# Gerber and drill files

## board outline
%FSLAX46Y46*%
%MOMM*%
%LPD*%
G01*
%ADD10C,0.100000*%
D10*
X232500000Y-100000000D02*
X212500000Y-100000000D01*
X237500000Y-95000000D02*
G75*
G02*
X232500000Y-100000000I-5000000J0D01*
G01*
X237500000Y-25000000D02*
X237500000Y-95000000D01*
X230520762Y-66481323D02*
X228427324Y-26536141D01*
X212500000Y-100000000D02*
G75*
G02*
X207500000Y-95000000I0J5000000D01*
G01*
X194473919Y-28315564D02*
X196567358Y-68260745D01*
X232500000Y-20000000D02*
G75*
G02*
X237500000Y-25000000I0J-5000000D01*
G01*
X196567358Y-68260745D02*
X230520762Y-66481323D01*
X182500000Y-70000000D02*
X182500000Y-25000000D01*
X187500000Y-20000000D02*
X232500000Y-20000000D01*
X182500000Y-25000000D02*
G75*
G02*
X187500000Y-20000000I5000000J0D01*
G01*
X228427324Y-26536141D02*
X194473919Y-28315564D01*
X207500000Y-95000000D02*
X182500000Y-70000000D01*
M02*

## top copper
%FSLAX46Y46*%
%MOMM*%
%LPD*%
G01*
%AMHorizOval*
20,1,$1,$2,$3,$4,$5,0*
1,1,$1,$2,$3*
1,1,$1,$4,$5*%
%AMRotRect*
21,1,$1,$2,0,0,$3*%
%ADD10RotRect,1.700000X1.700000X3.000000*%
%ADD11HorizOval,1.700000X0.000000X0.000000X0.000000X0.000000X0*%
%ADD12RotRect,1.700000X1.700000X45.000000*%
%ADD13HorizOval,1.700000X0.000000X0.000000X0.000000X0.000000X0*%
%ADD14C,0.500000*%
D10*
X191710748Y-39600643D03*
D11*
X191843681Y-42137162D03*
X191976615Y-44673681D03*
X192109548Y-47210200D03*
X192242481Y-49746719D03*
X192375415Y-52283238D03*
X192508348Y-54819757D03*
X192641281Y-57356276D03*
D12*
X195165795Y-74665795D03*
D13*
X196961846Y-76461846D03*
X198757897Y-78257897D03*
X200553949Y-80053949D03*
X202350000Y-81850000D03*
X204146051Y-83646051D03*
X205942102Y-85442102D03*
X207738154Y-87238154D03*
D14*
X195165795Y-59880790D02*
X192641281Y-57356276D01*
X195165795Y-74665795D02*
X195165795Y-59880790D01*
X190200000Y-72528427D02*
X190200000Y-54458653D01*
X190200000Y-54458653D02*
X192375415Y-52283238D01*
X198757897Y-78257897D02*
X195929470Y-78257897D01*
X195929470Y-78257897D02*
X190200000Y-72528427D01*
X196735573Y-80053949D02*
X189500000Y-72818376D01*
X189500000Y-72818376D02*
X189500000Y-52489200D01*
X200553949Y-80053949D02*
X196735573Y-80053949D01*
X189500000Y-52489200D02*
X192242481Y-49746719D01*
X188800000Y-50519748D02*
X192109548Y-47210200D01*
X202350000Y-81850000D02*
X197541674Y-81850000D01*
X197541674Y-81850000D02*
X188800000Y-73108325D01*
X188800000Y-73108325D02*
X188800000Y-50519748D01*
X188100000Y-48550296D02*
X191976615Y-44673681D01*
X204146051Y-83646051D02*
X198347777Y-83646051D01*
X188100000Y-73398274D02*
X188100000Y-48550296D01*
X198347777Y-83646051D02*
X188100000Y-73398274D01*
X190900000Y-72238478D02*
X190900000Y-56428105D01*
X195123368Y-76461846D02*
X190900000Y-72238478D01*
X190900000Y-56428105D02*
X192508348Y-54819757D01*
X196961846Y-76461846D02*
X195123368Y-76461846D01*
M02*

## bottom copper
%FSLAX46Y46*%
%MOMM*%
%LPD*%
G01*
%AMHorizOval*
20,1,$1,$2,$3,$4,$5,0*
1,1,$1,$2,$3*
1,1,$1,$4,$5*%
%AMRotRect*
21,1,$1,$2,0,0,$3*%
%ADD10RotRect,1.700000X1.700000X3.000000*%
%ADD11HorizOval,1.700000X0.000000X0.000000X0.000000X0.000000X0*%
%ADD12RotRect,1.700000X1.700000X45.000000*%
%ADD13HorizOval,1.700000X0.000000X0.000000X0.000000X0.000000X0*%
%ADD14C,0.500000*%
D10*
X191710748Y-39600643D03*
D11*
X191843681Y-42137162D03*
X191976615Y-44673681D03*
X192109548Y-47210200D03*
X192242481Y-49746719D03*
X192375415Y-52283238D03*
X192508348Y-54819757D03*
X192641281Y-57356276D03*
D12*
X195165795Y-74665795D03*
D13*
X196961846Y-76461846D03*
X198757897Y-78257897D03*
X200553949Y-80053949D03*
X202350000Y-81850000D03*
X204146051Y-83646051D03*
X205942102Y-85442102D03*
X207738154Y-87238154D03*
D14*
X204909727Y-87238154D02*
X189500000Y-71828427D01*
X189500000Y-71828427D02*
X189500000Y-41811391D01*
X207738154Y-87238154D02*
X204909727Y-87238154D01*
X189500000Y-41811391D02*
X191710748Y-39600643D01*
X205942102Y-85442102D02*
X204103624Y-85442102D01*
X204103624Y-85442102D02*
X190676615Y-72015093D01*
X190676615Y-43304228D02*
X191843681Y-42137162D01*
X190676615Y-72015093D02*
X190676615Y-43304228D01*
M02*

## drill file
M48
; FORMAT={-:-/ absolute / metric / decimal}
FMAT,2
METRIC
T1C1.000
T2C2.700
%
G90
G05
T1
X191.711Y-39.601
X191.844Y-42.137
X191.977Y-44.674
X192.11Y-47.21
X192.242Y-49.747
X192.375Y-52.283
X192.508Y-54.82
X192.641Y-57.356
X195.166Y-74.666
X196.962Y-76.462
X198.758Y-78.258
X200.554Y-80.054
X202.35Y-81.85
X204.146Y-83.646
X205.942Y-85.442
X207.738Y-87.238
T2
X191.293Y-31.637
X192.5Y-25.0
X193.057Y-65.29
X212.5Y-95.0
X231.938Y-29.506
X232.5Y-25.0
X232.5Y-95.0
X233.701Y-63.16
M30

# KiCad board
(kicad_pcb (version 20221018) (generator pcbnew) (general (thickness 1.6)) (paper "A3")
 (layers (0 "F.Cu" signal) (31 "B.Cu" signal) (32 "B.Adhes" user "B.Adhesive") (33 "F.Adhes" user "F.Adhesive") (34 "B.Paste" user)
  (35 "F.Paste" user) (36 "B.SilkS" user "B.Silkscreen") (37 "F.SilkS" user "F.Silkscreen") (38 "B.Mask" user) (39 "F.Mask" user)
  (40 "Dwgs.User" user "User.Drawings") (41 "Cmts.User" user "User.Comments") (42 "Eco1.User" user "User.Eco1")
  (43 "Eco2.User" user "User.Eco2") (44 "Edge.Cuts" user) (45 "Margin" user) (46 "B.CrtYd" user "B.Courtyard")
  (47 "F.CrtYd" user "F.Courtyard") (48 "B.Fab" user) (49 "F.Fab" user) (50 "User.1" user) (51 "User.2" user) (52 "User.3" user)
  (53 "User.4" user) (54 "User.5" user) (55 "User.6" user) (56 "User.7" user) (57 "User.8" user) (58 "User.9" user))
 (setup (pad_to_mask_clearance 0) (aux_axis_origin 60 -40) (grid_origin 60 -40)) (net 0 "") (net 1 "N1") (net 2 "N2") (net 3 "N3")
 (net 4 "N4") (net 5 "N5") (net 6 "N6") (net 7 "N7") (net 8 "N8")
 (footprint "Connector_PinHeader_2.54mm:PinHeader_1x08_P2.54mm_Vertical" (layer "F.Cu") (at 191.710748 39.600643 3)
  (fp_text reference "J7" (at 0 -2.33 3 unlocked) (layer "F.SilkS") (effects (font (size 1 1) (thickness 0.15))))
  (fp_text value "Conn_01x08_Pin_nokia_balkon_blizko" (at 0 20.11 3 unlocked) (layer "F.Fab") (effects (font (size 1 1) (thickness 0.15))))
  (pad "1" thru_hole rect (at 0 0 3) (size 1.7 1.7) (drill 1) (layers "*.Cu" "*.Mask") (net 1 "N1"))
  (pad "2" thru_hole oval (at 0 2.54 3) (size 1.7 1.7) (drill 1) (layers "*.Cu" "*.Mask") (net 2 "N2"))
  (pad "3" thru_hole oval (at 0 5.08 3) (size 1.7 1.7) (drill 1) (layers "*.Cu" "*.Mask") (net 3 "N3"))
  (pad "4" thru_hole oval (at 0 7.62 3) (size 1.7 1.7) (drill 1) (layers "*.Cu" "*.Mask") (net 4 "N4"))
  (pad "5" thru_hole oval (at 0 10.16 3) (size 1.7 1.7) (drill 1) (layers "*.Cu" "*.Mask") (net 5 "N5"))
  (pad "6" thru_hole oval (at 0 12.7 3) (size 1.7 1.7) (drill 1) (layers "*.Cu" "*.Mask") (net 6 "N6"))
  (pad "7" thru_hole oval (at 0 15.24 3) (size 1.7 1.7) (drill 1) (layers "*.Cu" "*.Mask") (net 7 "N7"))
  (pad "8" thru_hole oval (at 0 17.78 3) (size 1.7 1.7) (drill 1) (layers "*.Cu" "*.Mask") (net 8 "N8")))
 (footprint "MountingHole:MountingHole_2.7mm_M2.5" (layer "F.Cu") (at 232.5 25)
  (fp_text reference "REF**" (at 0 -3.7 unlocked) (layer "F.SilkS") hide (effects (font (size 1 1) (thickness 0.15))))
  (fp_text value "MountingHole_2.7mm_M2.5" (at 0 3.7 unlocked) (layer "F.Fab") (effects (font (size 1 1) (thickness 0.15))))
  (pad "" np_thru_hole circle (at 0 0) (size 2.7 2.7) (drill 2.7) (layers "*.Cu" "*.Mask")))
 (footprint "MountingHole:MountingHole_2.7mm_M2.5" (layer "F.Cu") (at 192.5 25)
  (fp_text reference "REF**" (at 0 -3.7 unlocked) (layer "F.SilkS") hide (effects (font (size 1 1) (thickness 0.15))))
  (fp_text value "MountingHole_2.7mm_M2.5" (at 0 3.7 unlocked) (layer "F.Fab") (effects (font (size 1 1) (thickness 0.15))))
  (pad "" np_thru_hole circle (at 0 0) (size 2.7 2.7) (drill 2.7) (layers "*.Cu" "*.Mask")))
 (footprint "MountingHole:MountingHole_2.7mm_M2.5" (layer "F.Cu") (at 191.293369 31.636572 3)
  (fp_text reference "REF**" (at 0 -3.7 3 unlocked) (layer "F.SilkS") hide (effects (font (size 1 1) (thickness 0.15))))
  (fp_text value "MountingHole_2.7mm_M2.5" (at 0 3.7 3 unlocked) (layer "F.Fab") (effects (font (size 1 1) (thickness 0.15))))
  (pad "" np_thru_hole circle (at 0 0 3) (size 2.7 2.7) (drill 2.7) (layers "*.Cu" "*.Mask")))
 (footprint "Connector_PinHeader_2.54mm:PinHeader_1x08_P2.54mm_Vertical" (layer "F.Cu") (at 195.165795 74.665795 45)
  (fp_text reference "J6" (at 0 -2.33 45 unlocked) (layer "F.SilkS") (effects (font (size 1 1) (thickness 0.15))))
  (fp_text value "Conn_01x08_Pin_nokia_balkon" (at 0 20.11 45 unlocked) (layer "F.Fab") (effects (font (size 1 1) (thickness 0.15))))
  (pad "1" thru_hole rect (at 0 0 45) (size 1.7 1.7) (drill 1) (layers "*.Cu" "*.Mask") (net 8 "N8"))
  (pad "2" thru_hole oval (at 0 2.54 45) (size 1.7 1.7) (drill 1) (layers "*.Cu" "*.Mask") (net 7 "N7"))
  (pad "3" thru_hole oval (at 0 5.08 45) (size 1.7 1.7) (drill 1) (layers "*.Cu" "*.Mask") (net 6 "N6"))
  (pad "4" thru_hole oval (at 0 7.62 45) (size 1.7 1.7) (drill 1) (layers "*.Cu" "*.Mask") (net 5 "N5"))
  (pad "5" thru_hole oval (at 0 10.16 45) (size 1.7 1.7) (drill 1) (layers "*.Cu" "*.Mask") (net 4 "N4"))
  (pad "6" thru_hole oval (at 0 12.7 45) (size 1.7 1.7) (drill 1) (layers "*.Cu" "*.Mask") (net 3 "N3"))
  (pad "7" thru_hole oval (at 0 15.24 45) (size 1.7 1.7) (drill 1) (layers "*.Cu" "*.Mask") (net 2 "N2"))
  (pad "8" thru_hole oval (at 0 17.78 45) (size 1.7 1.7) (drill 1) (layers "*.Cu" "*.Mask") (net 1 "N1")))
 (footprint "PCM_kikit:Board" (layer "F.Cu") (at 220.5 100 180)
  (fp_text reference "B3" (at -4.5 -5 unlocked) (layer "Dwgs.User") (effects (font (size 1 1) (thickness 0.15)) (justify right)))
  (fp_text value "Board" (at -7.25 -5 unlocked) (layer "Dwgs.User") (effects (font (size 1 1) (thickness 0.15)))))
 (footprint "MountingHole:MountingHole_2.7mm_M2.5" (layer "F.Cu") (at 232.5 95)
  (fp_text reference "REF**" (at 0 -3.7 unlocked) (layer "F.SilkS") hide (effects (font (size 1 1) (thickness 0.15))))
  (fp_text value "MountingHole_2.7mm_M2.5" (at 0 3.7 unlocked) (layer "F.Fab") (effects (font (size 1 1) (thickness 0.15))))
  (pad "" np_thru_hole circle (at 0 0) (size 2.7 2.7) (drill 2.7) (layers "*.Cu" "*.Mask")))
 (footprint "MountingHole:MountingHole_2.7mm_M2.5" (layer "F.Cu") (at 233.701313 63.160314 -177)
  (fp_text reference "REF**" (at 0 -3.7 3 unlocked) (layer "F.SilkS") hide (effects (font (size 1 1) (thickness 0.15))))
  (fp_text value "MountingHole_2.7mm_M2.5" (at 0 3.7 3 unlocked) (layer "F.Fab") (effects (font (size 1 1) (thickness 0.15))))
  (pad "" np_thru_hole circle (at 0 0 183) (size 2.7 2.7) (drill 2.7) (layers "*.Cu" "*.Mask")))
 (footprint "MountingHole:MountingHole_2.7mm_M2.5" (layer "F.Cu") (at 212.5 95)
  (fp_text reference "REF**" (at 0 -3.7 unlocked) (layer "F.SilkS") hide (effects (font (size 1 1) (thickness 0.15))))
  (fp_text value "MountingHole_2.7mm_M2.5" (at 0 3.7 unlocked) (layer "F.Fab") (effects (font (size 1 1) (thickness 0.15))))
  (pad "" np_thru_hole circle (at 0 0) (size 2.7 2.7) (drill 2.7) (layers "*.Cu" "*.Mask")))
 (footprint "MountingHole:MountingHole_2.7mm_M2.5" (layer "B.Cu") (at 193.05709 65.290388 3)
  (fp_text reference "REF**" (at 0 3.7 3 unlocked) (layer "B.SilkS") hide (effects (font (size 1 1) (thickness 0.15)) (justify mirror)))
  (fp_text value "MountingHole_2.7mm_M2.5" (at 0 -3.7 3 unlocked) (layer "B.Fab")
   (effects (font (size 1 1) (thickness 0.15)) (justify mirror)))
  (pad "" np_thru_hole circle (at 0 0 3) (size 2.7 2.7) (drill 2.7) (layers "*.Cu" "*.Mask")))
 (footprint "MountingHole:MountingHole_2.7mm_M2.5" (layer "B.Cu") (at 231.937591 29.506499 -177)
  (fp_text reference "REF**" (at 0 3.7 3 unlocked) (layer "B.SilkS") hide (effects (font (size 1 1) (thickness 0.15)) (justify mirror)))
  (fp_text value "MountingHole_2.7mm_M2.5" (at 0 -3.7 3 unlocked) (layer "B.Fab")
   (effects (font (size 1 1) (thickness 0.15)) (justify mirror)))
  (pad "" np_thru_hole circle (at 0 0 183) (size 2.7 2.7) (drill 2.7) (layers "*.Cu" "*.Mask")))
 (gr_line (start 232.5 100) (end 212.5 100) (stroke (width 0.1) (type default)) (layer "Edge.Cuts"))
 (gr_arc (start 237.5 95) (mid 236.035533 98.535533) (end 232.5 100) (stroke (width 0.1) (type default)) (layer "Edge.Cuts"))
 (gr_line (start 237.5 25) (end 237.5 95) (stroke (width 0.1) (type default)) (layer "Edge.Cuts"))
 (gr_line (start 230.520762 66.481323) (end 228.427324 26.536141) (stroke (width 0.1) (type default)) (layer "Edge.Cuts"))
 (gr_arc (start 212.5 100) (mid 208.964466 98.535533) (end 207.5 95) (stroke (width 0.1) (type default)) (layer "Edge.Cuts"))
 (gr_line (start 194.473919 28.315564) (end 196.567358 68.260745) (stroke (width 0.1) (type default)) (layer "Edge.Cuts"))
 (gr_arc (start 232.5 20) (mid 236.035533 21.464466) (end 237.5 25) (stroke (width 0.1) (type default)) (layer "Edge.Cuts"))
 (gr_line (start 196.567358 68.260745) (end 230.520762 66.481323) (stroke (width 0.1) (type default)) (layer "Edge.Cuts"))
 (gr_line (start 182.5 70) (end 182.5 25) (stroke (width 0.1) (type default)) (layer "Edge.Cuts"))
 (gr_line (start 187.5 20) (end 232.5 20) (stroke (width 0.1) (type default)) (layer "Edge.Cuts"))
 (gr_arc (start 182.5 25) (mid 183.964466 21.464466) (end 187.5 20) (stroke (width 0.1) (type default)) (layer "Edge.Cuts"))
 (gr_line (start 228.427324 26.536141) (end 194.473919 28.315564) (stroke (width 0.1) (type default)) (layer "Edge.Cuts"))
 (gr_line (start 207.5 95) (end 182.5 70) (stroke (width 0.1) (type default)) (layer "Edge.Cuts"))
 (segment (start 204.909727 87.238154) (end 189.5 71.828427) (width 0.5) (layer "B.Cu") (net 1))
 (segment (start 189.5 71.828427) (end 189.5 41.811391) (width 0.5) (layer "B.Cu") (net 1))
 (segment (start 207.738154 87.238154) (end 204.909727 87.238154) (width 0.5) (layer "B.Cu") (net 1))
 (segment (start 189.5 41.811391) (end 191.710748 39.600643) (width 0.5) (layer "B.Cu") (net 1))
 (segment (start 195.165795 59.88079) (end 192.641281 57.356276) (width 0.5) (layer "F.Cu") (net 8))
 (segment (start 195.165795 74.665795) (end 195.165795 59.88079) (width 0.5) (layer "F.Cu") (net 8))
 (segment (start 190.2 72.528427) (end 190.2 54.458653) (width 0.5) (layer "F.Cu") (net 6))
 (segment (start 190.2 54.458653) (end 192.375415 52.283238) (width 0.5) (layer "F.Cu") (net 6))
 (segment (start 198.757897 78.257897) (end 195.92947 78.257897) (width 0.5) (layer "F.Cu") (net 6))
 (segment (start 195.92947 78.257897) (end 190.2 72.528427) (width 0.5) (layer "F.Cu") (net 6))
 (segment (start 196.735573 80.053949) (end 189.5 72.818376) (width 0.5) (layer "F.Cu") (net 5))
 (segment (start 189.5 72.818376) (end 189.5 52.4892) (width 0.5) (layer "F.Cu") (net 5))
 (segment (start 200.553949 80.053949) (end 196.735573 80.053949) (width 0.5) (layer "F.Cu") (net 5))
 (segment (start 189.5 52.4892) (end 192.242481 49.746719) (width 0.5) (layer "F.Cu") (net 5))
 (segment (start 188.8 50.519748) (end 192.109548 47.2102) (width 0.5) (layer "F.Cu") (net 4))
 (segment (start 202.35 81.85) (end 197.541674 81.85) (width 0.5) (layer "F.Cu") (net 4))
 (segment (start 197.541674 81.85) (end 188.8 73.108325) (width 0.5) (layer "F.Cu") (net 4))
 (segment (start 188.8 73.108325) (end 188.8 50.519748) (width 0.5) (layer "F.Cu") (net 4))
 (segment (start 188.1 48.550296) (end 191.976615 44.673681) (width 0.5) (layer "F.Cu") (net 3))
 (segment (start 204.146051 83.646051) (end 198.347777 83.646051) (width 0.5) (layer "F.Cu") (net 3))
 (segment (start 188.1 73.398274) (end 188.1 48.550296) (width 0.5) (layer "F.Cu") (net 3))
 (segment (start 198.347777 83.646051) (end 188.1 73.398274) (width 0.5) (layer "F.Cu") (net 3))
 (segment (start 205.942102 85.442102) (end 204.103624 85.442102) (width 0.5) (layer "B.Cu") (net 2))
 (segment (start 204.103624 85.442102) (end 190.676615 72.015093) (width 0.5) (layer "B.Cu") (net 2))
 (segment (start 190.676615 43.304228) (end 191.843681 42.137162) (width 0.5) (layer "B.Cu") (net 2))
 (segment (start 190.676615 72.015093) (end 190.676615 43.304228) (width 0.5) (layer "B.Cu") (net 2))
 (segment (start 190.9 72.238478) (end 190.9 56.428105) (width 0.5) (layer "F.Cu") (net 7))
 (segment (start 195.123368 76.461846) (end 190.9 72.238478) (width 0.5) (layer "F.Cu") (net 7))
 (segment (start 190.9 56.428105) (end 192.508348 54.819757) (width 0.5) (layer "F.Cu") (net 7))
 (segment (start 196.961846 76.461846) (end 195.123368 76.461846) (width 0.5) (layer "F.Cu") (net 7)))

